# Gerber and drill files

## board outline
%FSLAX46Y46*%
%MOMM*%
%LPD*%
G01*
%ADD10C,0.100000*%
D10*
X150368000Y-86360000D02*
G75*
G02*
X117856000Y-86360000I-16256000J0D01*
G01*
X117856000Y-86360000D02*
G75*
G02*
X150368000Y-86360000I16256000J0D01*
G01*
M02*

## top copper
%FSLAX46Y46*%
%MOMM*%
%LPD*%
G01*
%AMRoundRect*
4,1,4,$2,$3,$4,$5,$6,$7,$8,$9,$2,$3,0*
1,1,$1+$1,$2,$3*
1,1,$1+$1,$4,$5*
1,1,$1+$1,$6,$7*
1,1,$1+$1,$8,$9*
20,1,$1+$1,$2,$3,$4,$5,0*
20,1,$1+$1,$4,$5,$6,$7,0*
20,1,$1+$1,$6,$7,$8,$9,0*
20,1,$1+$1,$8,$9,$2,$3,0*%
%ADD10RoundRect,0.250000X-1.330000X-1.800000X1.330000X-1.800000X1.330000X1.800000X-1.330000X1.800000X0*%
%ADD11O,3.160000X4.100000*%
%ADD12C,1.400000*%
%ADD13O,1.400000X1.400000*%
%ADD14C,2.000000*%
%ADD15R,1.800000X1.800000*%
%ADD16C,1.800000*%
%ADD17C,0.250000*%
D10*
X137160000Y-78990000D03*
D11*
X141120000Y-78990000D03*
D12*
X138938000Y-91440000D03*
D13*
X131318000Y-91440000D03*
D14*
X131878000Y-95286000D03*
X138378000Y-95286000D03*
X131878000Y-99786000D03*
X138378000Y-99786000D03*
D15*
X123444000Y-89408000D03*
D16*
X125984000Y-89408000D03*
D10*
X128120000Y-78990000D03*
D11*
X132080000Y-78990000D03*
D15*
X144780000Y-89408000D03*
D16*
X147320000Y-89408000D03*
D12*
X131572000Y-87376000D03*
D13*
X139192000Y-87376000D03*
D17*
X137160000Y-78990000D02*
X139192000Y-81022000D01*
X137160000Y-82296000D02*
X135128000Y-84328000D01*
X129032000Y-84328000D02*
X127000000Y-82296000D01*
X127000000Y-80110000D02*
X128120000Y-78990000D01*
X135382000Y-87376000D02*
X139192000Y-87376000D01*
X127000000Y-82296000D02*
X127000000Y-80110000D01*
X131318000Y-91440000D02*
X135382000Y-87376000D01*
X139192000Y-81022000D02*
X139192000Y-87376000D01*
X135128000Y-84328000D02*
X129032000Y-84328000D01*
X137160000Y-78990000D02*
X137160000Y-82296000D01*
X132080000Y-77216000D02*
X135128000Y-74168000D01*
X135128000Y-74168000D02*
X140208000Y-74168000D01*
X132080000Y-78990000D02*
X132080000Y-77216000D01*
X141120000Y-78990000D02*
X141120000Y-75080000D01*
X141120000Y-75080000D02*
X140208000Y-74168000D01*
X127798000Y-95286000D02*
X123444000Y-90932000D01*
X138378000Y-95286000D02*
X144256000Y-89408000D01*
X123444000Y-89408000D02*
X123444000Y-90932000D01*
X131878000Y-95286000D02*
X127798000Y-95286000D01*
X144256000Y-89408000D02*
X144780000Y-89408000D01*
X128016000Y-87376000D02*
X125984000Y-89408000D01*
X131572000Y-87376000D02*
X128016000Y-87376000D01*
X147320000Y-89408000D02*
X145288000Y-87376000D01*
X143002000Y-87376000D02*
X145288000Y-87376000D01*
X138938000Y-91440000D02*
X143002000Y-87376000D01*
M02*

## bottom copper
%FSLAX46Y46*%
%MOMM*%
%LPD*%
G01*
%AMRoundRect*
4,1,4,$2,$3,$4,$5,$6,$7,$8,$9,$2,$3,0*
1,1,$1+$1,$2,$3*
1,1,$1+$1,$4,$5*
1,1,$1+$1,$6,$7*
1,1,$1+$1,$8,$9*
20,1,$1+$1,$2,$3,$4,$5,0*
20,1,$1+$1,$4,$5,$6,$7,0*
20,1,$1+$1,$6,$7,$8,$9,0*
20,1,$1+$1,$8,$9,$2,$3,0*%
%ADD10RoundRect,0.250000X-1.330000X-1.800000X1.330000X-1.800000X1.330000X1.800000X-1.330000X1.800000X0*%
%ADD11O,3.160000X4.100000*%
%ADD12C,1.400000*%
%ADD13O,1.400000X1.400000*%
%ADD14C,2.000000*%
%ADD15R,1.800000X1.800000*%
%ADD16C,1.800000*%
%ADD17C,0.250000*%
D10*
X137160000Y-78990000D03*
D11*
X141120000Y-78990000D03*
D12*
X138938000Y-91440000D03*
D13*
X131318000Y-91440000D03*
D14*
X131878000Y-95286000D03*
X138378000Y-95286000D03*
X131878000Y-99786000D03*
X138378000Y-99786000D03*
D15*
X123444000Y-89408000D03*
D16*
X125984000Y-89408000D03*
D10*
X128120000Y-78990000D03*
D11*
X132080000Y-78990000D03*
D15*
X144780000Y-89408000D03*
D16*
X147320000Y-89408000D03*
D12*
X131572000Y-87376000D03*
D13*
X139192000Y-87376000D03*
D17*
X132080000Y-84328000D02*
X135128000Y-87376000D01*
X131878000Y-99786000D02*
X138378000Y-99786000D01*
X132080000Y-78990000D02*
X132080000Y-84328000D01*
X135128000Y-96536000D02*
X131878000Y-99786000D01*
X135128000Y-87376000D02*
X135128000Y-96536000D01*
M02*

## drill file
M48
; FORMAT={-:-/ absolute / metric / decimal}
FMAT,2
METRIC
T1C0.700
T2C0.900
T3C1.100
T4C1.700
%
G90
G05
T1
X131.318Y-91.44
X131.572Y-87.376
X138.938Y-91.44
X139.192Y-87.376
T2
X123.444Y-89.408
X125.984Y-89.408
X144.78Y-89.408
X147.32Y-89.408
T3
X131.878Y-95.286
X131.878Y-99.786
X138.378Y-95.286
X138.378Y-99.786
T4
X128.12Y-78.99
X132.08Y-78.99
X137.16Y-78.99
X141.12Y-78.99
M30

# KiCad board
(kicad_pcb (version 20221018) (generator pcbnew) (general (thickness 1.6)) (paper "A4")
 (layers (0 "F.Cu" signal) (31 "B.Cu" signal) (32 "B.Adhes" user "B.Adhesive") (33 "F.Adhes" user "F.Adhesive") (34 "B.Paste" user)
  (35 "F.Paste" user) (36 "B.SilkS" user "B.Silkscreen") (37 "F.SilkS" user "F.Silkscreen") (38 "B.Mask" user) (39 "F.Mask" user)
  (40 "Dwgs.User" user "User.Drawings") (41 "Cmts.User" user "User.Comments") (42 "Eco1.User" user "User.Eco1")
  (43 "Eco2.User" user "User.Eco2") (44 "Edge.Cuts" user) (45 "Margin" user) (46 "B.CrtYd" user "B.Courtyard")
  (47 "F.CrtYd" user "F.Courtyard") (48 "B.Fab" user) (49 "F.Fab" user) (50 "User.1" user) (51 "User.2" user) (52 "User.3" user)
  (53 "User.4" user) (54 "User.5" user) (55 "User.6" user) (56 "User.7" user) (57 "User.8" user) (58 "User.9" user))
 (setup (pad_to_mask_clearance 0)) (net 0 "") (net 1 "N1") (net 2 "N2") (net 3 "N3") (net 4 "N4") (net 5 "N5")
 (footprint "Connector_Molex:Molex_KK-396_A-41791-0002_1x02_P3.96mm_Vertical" (layer "F.Cu") (at 137.16 78.99)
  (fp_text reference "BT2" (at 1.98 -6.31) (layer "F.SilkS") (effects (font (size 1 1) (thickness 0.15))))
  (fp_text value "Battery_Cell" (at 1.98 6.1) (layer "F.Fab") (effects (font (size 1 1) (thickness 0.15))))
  (pad "1" thru_hole roundrect (at 0 0) (size 3.16 4.1) (drill 1.7) (layers "*.Cu" "*.Mask") (roundrect_rratio 0.079114) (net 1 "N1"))
  (pad "2" thru_hole oval (at 3.96 0) (size 3.16 4.1) (drill 1.7) (layers "*.Cu" "*.Mask") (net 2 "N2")))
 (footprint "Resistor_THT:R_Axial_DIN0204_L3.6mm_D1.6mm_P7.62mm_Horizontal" (layer "F.Cu") (at 138.938 91.44 180)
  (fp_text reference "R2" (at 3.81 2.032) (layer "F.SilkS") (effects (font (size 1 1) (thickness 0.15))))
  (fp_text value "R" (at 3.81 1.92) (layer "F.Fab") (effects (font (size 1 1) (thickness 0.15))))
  (pad "1" thru_hole circle (at 0 0 180) (size 1.4 1.4) (drill 0.7) (layers "*.Cu" "*.Mask") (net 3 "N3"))
  (pad "2" thru_hole oval (at 7.62 0 180) (size 1.4 1.4) (drill 0.7) (layers "*.Cu" "*.Mask") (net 1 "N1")))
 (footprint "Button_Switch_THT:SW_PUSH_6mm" (layer "F.Cu") (at 131.878 95.286)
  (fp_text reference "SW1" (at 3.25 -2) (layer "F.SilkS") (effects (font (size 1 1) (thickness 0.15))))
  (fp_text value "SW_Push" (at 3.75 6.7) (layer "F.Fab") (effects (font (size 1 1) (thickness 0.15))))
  (pad "1" thru_hole circle (at 0 0 90) (size 2 2) (drill 1.1) (layers "*.Cu" "*.Mask") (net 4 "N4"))
  (pad "1" thru_hole circle (at 6.5 0 90) (size 2 2) (drill 1.1) (layers "*.Cu" "*.Mask") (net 4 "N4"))
  (pad "2" thru_hole circle (at 0 4.5 90) (size 2 2) (drill 1.1) (layers "*.Cu" "*.Mask") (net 2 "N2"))
  (pad "2" thru_hole circle (at 6.5 4.5 90) (size 2 2) (drill 1.1) (layers "*.Cu" "*.Mask") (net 2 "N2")))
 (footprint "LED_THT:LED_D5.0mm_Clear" (layer "F.Cu") (at 123.444 89.408)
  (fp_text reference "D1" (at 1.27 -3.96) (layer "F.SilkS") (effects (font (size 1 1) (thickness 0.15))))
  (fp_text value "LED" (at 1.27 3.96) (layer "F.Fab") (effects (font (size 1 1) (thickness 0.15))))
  (pad "1" thru_hole rect (at 0 0) (size 1.8 1.8) (drill 0.9) (layers "*.Cu" "*.Mask") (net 4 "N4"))
  (pad "2" thru_hole circle (at 2.54 0) (size 1.8 1.8) (drill 0.9) (layers "*.Cu" "*.Mask") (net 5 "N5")))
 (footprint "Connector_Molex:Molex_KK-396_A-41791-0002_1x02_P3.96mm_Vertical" (layer "F.Cu") (at 128.12 78.99)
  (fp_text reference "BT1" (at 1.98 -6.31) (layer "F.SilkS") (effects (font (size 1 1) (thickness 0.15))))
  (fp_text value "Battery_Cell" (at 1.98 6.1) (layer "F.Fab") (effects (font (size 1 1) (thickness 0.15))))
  (pad "1" thru_hole roundrect (at 0 0) (size 3.16 4.1) (drill 1.7) (layers "*.Cu" "*.Mask") (roundrect_rratio 0.079114) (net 1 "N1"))
  (pad "2" thru_hole oval (at 3.96 0) (size 3.16 4.1) (drill 1.7) (layers "*.Cu" "*.Mask") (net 2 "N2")))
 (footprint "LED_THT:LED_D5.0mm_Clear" (layer "F.Cu") (at 144.78 89.408)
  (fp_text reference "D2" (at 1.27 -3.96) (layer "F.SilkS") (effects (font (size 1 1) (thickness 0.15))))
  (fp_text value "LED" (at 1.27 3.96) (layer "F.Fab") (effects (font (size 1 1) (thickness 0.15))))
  (pad "1" thru_hole rect (at 0 0) (size 1.8 1.8) (drill 0.9) (layers "*.Cu" "*.Mask") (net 4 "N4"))
  (pad "2" thru_hole circle (at 2.54 0) (size 1.8 1.8) (drill 0.9) (layers "*.Cu" "*.Mask") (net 3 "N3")))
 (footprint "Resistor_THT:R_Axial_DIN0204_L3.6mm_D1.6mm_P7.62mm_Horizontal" (layer "F.Cu") (at 131.572 87.376)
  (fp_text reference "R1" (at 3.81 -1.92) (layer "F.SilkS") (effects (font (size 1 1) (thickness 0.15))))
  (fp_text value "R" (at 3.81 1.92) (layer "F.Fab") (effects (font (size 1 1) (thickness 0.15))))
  (pad "1" thru_hole circle (at 0 0) (size 1.4 1.4) (drill 0.7) (layers "*.Cu" "*.Mask") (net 5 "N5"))
  (pad "2" thru_hole oval (at 7.62 0) (size 1.4 1.4) (drill 0.7) (layers "*.Cu" "*.Mask") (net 1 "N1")))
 (gr_circle (center 134.112 86.36) (end 150.368 86.36) (stroke (width 0.1) (type default)) (fill none) (layer "Edge.Cuts"))
 (segment (start 137.16 78.99) (end 139.192 81.022) (width 0.25) (layer "F.Cu") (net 1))
 (segment (start 137.16 82.296) (end 135.128 84.328) (width 0.25) (layer "F.Cu") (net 1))
 (segment (start 129.032 84.328) (end 127 82.296) (width 0.25) (layer "F.Cu") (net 1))
 (segment (start 127 80.11) (end 128.12 78.99) (width 0.25) (layer "F.Cu") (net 1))
 (segment (start 135.382 87.376) (end 139.192 87.376) (width 0.25) (layer "F.Cu") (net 1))
 (segment (start 127 82.296) (end 127 80.11) (width 0.25) (layer "F.Cu") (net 1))
 (segment (start 131.318 91.44) (end 135.382 87.376) (width 0.25) (layer "F.Cu") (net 1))
 (segment (start 139.192 81.022) (end 139.192 87.376) (width 0.25) (layer "F.Cu") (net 1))
 (segment (start 135.128 84.328) (end 129.032 84.328) (width 0.25) (layer "F.Cu") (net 1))
 (segment (start 137.16 78.99) (end 137.16 82.296) (width 0.25) (layer "F.Cu") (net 1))
 (segment (start 132.08 77.216) (end 135.128 74.168) (width 0.25) (layer "F.Cu") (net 2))
 (segment (start 135.128 74.168) (end 140.208 74.168) (width 0.25) (layer "F.Cu") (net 2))
 (segment (start 132.08 78.99) (end 132.08 77.216) (width 0.25) (layer "F.Cu") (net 2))
 (segment (start 141.12 78.99) (end 141.12 75.08) (width 0.25) (layer "F.Cu") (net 2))
 (segment (start 141.12 75.08) (end 140.208 74.168) (width 0.25) (layer "F.Cu") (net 2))
 (segment (start 132.08 84.328) (end 135.128 87.376) (width 0.25) (layer "B.Cu") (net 2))
 (segment (start 131.878 99.786) (end 138.378 99.786) (width 0.25) (layer "B.Cu") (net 2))
 (segment (start 132.08 78.99) (end 132.08 84.328) (width 0.25) (layer "B.Cu") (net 2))
 (segment (start 135.128 96.536) (end 131.878 99.786) (width 0.25) (layer "B.Cu") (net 2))
 (segment (start 135.128 87.376) (end 135.128 96.536) (width 0.25) (layer "B.Cu") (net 2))
 (segment (start 127.798 95.286) (end 123.444 90.932) (width 0.25) (layer "F.Cu") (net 4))
 (segment (start 138.378 95.286) (end 144.256 89.408) (width 0.25) (layer "F.Cu") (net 4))
 (segment (start 123.444 89.408) (end 123.444 90.932) (width 0.25) (layer "F.Cu") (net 4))
 (segment (start 131.878 95.286) (end 127.798 95.286) (width 0.25) (layer "F.Cu") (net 4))
 (segment (start 144.256 89.408) (end 144.78 89.408) (width 0.25) (layer "F.Cu") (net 4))
 (segment (start 128.016 87.376) (end 125.984 89.408) (width 0.25) (layer "F.Cu") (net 5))
 (segment (start 131.572 87.376) (end 128.016 87.376) (width 0.25) (layer "F.Cu") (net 5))
 (segment (start 147.32 89.408) (end 145.288 87.376) (width 0.25) (layer "F.Cu") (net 3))
 (segment (start 143.002 87.376) (end 145.288 87.376) (width 0.25) (layer "F.Cu") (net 3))
 (segment (start 138.938 91.44) (end 143.002 87.376) (width 0.25) (layer "F.Cu") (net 3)))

